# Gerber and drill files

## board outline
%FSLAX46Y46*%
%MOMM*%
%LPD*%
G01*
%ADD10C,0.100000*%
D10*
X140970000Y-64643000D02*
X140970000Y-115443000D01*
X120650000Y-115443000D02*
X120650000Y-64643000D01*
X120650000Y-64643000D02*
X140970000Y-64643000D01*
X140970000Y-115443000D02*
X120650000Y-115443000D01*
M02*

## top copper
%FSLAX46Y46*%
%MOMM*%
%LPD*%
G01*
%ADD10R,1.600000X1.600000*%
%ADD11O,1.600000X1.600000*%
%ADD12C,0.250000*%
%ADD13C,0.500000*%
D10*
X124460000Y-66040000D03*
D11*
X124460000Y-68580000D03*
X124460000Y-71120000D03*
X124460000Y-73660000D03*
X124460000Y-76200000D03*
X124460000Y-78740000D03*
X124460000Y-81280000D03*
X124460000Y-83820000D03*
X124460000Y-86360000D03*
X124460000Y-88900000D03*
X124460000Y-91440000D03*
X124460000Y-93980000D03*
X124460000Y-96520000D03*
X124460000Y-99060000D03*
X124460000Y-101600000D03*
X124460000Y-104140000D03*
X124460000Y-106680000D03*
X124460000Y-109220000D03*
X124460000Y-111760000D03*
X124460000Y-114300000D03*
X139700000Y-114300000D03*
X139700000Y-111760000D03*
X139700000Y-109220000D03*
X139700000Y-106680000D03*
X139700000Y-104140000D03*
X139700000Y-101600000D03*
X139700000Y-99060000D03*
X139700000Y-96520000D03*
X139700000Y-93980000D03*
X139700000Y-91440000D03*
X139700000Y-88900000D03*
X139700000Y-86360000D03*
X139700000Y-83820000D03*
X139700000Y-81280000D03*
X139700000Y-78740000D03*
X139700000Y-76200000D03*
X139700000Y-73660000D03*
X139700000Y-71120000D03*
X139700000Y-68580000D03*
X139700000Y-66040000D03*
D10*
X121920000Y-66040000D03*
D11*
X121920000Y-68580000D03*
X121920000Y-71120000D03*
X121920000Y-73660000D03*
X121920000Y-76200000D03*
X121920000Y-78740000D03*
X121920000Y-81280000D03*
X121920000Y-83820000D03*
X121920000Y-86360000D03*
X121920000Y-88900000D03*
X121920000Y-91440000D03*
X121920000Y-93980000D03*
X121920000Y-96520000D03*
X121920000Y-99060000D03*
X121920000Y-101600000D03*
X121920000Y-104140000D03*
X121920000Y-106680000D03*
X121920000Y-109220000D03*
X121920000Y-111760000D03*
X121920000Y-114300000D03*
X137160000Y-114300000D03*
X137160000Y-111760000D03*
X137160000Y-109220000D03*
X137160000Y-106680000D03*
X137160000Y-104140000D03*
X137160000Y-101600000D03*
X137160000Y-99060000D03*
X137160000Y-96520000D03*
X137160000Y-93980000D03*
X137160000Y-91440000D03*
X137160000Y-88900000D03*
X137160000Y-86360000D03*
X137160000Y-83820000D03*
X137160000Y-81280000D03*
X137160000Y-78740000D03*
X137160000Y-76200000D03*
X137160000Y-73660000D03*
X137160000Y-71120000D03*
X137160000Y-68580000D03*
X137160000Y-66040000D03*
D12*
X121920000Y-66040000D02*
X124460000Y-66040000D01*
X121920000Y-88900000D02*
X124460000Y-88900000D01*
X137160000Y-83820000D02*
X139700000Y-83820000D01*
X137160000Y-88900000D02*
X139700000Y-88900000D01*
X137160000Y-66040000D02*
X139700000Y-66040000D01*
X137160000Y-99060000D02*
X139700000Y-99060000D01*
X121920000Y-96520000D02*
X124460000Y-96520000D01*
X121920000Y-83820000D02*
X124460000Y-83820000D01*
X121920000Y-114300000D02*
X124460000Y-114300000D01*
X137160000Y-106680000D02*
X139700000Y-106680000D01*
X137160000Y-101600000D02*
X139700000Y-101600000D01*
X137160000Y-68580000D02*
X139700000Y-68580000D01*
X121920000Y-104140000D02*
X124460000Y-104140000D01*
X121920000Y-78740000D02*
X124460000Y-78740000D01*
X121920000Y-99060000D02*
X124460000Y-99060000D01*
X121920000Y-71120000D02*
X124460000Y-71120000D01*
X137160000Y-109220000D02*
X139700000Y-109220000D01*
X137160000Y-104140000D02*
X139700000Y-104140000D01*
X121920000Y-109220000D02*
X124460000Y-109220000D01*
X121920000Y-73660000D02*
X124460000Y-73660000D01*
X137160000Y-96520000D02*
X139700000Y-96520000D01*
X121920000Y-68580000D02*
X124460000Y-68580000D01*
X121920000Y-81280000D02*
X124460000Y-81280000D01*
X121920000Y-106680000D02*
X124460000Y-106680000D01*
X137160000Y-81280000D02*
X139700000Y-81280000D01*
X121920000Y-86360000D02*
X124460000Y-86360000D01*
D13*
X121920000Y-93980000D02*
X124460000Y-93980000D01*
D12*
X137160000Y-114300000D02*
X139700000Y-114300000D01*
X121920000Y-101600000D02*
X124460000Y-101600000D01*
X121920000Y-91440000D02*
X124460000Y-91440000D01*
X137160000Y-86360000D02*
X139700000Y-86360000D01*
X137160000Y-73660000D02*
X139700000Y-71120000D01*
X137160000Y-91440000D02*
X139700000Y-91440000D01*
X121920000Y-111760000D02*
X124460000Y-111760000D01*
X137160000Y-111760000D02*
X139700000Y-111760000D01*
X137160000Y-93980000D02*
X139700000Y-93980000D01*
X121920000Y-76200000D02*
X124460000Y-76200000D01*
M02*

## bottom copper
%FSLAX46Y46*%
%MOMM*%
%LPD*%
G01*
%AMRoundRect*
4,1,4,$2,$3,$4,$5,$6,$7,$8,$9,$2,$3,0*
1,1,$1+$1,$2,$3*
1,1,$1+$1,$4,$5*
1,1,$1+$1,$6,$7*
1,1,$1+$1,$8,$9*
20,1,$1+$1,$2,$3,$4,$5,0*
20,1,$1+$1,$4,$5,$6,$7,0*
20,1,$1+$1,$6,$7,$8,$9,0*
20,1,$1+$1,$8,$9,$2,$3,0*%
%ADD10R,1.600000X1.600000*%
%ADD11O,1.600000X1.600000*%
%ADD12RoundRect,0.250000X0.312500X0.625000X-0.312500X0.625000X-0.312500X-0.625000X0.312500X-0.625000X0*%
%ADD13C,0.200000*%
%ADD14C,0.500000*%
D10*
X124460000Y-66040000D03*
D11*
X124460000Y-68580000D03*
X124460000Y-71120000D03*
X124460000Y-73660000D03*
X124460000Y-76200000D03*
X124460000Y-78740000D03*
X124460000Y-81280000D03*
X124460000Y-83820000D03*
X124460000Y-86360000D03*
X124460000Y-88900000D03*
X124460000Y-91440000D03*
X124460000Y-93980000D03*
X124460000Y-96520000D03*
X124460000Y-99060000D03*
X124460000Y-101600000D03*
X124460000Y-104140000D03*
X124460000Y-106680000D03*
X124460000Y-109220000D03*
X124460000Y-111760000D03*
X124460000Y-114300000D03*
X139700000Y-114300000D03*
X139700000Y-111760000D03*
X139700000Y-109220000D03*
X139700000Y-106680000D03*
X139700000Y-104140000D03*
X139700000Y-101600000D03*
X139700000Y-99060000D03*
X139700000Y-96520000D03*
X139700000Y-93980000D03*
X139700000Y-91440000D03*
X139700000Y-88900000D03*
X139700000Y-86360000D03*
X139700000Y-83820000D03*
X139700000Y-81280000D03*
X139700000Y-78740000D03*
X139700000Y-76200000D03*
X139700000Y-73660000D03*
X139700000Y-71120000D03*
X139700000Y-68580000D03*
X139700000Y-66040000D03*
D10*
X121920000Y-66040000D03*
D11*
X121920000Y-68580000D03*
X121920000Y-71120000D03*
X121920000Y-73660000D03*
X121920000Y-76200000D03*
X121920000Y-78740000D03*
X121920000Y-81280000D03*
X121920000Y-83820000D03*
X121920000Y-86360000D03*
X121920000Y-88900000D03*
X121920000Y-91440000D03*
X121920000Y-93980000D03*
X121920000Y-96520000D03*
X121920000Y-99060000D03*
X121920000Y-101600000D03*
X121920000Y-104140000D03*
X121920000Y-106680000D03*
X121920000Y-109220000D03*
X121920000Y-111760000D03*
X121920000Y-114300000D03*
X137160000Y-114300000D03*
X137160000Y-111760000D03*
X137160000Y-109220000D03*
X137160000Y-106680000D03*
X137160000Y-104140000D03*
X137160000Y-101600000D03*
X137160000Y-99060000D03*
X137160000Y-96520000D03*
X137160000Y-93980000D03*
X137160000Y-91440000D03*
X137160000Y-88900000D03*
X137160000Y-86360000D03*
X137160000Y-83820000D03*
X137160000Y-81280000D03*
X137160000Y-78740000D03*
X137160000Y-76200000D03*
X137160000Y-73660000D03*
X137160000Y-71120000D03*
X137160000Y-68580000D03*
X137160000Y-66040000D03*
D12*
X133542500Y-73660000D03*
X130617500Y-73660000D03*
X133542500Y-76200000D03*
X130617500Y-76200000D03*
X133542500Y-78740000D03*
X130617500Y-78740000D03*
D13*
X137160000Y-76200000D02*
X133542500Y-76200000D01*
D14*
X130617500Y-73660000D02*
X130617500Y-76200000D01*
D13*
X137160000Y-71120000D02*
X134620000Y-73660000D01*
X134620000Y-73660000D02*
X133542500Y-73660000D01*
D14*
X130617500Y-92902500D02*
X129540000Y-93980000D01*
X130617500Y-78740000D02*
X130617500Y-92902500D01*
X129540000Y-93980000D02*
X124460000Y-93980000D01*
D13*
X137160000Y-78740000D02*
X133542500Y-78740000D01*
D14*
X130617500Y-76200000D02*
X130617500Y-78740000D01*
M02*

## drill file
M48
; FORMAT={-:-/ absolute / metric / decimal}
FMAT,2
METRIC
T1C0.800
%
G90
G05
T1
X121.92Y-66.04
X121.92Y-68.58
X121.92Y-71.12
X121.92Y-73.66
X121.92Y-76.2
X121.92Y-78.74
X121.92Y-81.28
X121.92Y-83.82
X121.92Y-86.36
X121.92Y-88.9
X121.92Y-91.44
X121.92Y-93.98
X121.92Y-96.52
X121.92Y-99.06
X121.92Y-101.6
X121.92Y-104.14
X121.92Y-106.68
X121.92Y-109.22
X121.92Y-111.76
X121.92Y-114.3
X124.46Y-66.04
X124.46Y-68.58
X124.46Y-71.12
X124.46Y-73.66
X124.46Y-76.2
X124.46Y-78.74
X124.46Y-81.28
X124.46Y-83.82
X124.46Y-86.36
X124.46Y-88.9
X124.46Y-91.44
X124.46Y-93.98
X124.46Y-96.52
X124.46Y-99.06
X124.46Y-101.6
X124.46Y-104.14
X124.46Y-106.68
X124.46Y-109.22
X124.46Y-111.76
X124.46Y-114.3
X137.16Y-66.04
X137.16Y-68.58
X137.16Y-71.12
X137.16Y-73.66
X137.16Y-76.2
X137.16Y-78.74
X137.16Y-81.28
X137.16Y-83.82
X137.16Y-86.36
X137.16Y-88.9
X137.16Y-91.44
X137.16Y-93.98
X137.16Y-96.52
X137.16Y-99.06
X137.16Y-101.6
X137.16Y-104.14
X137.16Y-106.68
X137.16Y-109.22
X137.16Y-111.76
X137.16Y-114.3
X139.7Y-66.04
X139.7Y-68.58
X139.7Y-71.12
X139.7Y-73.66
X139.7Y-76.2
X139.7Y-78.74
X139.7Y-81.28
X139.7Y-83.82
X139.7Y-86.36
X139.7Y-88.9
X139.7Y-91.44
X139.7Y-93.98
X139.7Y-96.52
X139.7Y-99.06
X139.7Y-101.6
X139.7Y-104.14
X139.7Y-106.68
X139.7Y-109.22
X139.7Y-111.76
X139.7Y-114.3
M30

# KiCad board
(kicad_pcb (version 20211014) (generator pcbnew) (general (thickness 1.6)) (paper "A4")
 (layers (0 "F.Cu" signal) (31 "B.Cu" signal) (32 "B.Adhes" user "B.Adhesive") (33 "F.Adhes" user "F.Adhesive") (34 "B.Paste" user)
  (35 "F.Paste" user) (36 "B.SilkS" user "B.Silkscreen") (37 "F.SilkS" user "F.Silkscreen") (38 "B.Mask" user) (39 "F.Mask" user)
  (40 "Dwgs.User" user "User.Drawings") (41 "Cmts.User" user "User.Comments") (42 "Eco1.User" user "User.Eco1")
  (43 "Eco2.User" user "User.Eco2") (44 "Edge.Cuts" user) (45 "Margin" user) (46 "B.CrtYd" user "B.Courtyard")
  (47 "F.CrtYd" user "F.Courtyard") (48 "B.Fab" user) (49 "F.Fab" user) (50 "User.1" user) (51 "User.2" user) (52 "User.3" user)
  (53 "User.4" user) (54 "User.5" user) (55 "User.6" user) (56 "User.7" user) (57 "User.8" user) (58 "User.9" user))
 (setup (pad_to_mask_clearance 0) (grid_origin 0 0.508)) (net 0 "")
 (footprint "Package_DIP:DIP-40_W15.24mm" (layer "F.Cu") (at 124.46 66.04)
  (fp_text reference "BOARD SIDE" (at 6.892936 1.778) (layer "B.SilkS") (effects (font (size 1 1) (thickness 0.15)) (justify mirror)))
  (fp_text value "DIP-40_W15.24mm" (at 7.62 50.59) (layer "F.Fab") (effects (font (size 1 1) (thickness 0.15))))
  (pad "1" thru_hole rect (at 0 0) (size 1.6 1.6) (drill 0.8) (layers *.Cu *.Mask))
  (pad "2" thru_hole oval (at 0 2.54) (size 1.6 1.6) (drill 0.8) (layers *.Cu *.Mask))
  (pad "3" thru_hole oval (at 0 5.08) (size 1.6 1.6) (drill 0.8) (layers *.Cu *.Mask))
  (pad "4" thru_hole oval (at 0 7.62) (size 1.6 1.6) (drill 0.8) (layers *.Cu *.Mask))
  (pad "5" thru_hole oval (at 0 10.16) (size 1.6 1.6) (drill 0.8) (layers *.Cu *.Mask))
  (pad "6" thru_hole oval (at 0 12.7) (size 1.6 1.6) (drill 0.8) (layers *.Cu *.Mask))
  (pad "7" thru_hole oval (at 0 15.24) (size 1.6 1.6) (drill 0.8) (layers *.Cu *.Mask))
  (pad "8" thru_hole oval (at 0 17.78) (size 1.6 1.6) (drill 0.8) (layers *.Cu *.Mask))
  (pad "9" thru_hole oval (at 0 20.32) (size 1.6 1.6) (drill 0.8) (layers *.Cu *.Mask))
  (pad "10" thru_hole oval (at 0 22.86) (size 1.6 1.6) (drill 0.8) (layers *.Cu *.Mask))
  (pad "11" thru_hole oval (at 0 25.4) (size 1.6 1.6) (drill 0.8) (layers *.Cu *.Mask))
  (pad "12" thru_hole oval (at 0 27.94) (size 1.6 1.6) (drill 0.8) (layers *.Cu *.Mask))
  (pad "13" thru_hole oval (at 0 30.48) (size 1.6 1.6) (drill 0.8) (layers *.Cu *.Mask))
  (pad "14" thru_hole oval (at 0 33.02) (size 1.6 1.6) (drill 0.8) (layers *.Cu *.Mask))
  (pad "15" thru_hole oval (at 0 35.56) (size 1.6 1.6) (drill 0.8) (layers *.Cu *.Mask))
  (pad "16" thru_hole oval (at 0 38.1) (size 1.6 1.6) (drill 0.8) (layers *.Cu *.Mask))
  (pad "17" thru_hole oval (at 0 40.64) (size 1.6 1.6) (drill 0.8) (layers *.Cu *.Mask))
  (pad "18" thru_hole oval (at 0 43.18) (size 1.6 1.6) (drill 0.8) (layers *.Cu *.Mask))
  (pad "19" thru_hole oval (at 0 45.72) (size 1.6 1.6) (drill 0.8) (layers *.Cu *.Mask))
  (pad "20" thru_hole oval (at 0 48.26) (size 1.6 1.6) (drill 0.8) (layers *.Cu *.Mask))
  (pad "21" thru_hole oval (at 15.24 48.26) (size 1.6 1.6) (drill 0.8) (layers *.Cu *.Mask))
  (pad "22" thru_hole oval (at 15.24 45.72) (size 1.6 1.6) (drill 0.8) (layers *.Cu *.Mask))
  (pad "23" thru_hole oval (at 15.24 43.18) (size 1.6 1.6) (drill 0.8) (layers *.Cu *.Mask))
  (pad "24" thru_hole oval (at 15.24 40.64) (size 1.6 1.6) (drill 0.8) (layers *.Cu *.Mask))
  (pad "25" thru_hole oval (at 15.24 38.1) (size 1.6 1.6) (drill 0.8) (layers *.Cu *.Mask))
  (pad "26" thru_hole oval (at 15.24 35.56) (size 1.6 1.6) (drill 0.8) (layers *.Cu *.Mask))
  (pad "27" thru_hole oval (at 15.24 33.02) (size 1.6 1.6) (drill 0.8) (layers *.Cu *.Mask))
  (pad "28" thru_hole oval (at 15.24 30.48) (size 1.6 1.6) (drill 0.8) (layers *.Cu *.Mask))
  (pad "29" thru_hole oval (at 15.24 27.94) (size 1.6 1.6) (drill 0.8) (layers *.Cu *.Mask))
  (pad "30" thru_hole oval (at 15.24 25.4) (size 1.6 1.6) (drill 0.8) (layers *.Cu *.Mask))
  (pad "31" thru_hole oval (at 15.24 22.86) (size 1.6 1.6) (drill 0.8) (layers *.Cu *.Mask))
  (pad "32" thru_hole oval (at 15.24 20.32) (size 1.6 1.6) (drill 0.8) (layers *.Cu *.Mask))
  (pad "33" thru_hole oval (at 15.24 17.78) (size 1.6 1.6) (drill 0.8) (layers *.Cu *.Mask))
  (pad "34" thru_hole oval (at 15.24 15.24) (size 1.6 1.6) (drill 0.8) (layers *.Cu *.Mask))
  (pad "35" thru_hole oval (at 15.24 12.7) (size 1.6 1.6) (drill 0.8) (layers *.Cu *.Mask))
  (pad "36" thru_hole oval (at 15.24 10.16) (size 1.6 1.6) (drill 0.8) (layers *.Cu *.Mask))
  (pad "37" thru_hole oval (at 15.24 7.62) (size 1.6 1.6) (drill 0.8) (layers *.Cu *.Mask))
  (pad "38" thru_hole oval (at 15.24 5.08) (size 1.6 1.6) (drill 0.8) (layers *.Cu *.Mask))
  (pad "39" thru_hole oval (at 15.24 2.54) (size 1.6 1.6) (drill 0.8) (layers *.Cu *.Mask))
  (pad "40" thru_hole oval (at 15.24 0) (size 1.6 1.6) (drill 0.8) (layers *.Cu *.Mask)))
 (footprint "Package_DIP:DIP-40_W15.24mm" (layer "F.Cu") (at 121.92 66.04)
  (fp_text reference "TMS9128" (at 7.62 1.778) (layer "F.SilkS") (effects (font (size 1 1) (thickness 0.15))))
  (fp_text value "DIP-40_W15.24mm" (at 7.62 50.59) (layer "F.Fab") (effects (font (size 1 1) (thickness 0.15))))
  (pad "1" thru_hole rect (at 0 0) (size 1.6 1.6) (drill 0.8) (layers *.Cu *.Mask))
  (pad "2" thru_hole oval (at 0 2.54) (size 1.6 1.6) (drill 0.8) (layers *.Cu *.Mask))
  (pad "3" thru_hole oval (at 0 5.08) (size 1.6 1.6) (drill 0.8) (layers *.Cu *.Mask))
  (pad "4" thru_hole oval (at 0 7.62) (size 1.6 1.6) (drill 0.8) (layers *.Cu *.Mask))
  (pad "5" thru_hole oval (at 0 10.16) (size 1.6 1.6) (drill 0.8) (layers *.Cu *.Mask))
  (pad "6" thru_hole oval (at 0 12.7) (size 1.6 1.6) (drill 0.8) (layers *.Cu *.Mask))
  (pad "7" thru_hole oval (at 0 15.24) (size 1.6 1.6) (drill 0.8) (layers *.Cu *.Mask))
  (pad "8" thru_hole oval (at 0 17.78) (size 1.6 1.6) (drill 0.8) (layers *.Cu *.Mask))
  (pad "9" thru_hole oval (at 0 20.32) (size 1.6 1.6) (drill 0.8) (layers *.Cu *.Mask))
  (pad "10" thru_hole oval (at 0 22.86) (size 1.6 1.6) (drill 0.8) (layers *.Cu *.Mask))
  (pad "11" thru_hole oval (at 0 25.4) (size 1.6 1.6) (drill 0.8) (layers *.Cu *.Mask))
  (pad "12" thru_hole oval (at 0 27.94) (size 1.6 1.6) (drill 0.8) (layers *.Cu *.Mask))
  (pad "13" thru_hole oval (at 0 30.48) (size 1.6 1.6) (drill 0.8) (layers *.Cu *.Mask))
  (pad "14" thru_hole oval (at 0 33.02) (size 1.6 1.6) (drill 0.8) (layers *.Cu *.Mask))
  (pad "15" thru_hole oval (at 0 35.56) (size 1.6 1.6) (drill 0.8) (layers *.Cu *.Mask))
  (pad "16" thru_hole oval (at 0 38.1) (size 1.6 1.6) (drill 0.8) (layers *.Cu *.Mask))
  (pad "17" thru_hole oval (at 0 40.64) (size 1.6 1.6) (drill 0.8) (layers *.Cu *.Mask))
  (pad "18" thru_hole oval (at 0 43.18) (size 1.6 1.6) (drill 0.8) (layers *.Cu *.Mask))
  (pad "19" thru_hole oval (at 0 45.72) (size 1.6 1.6) (drill 0.8) (layers *.Cu *.Mask))
  (pad "20" thru_hole oval (at 0 48.26) (size 1.6 1.6) (drill 0.8) (layers *.Cu *.Mask))
  (pad "21" thru_hole oval (at 15.24 48.26) (size 1.6 1.6) (drill 0.8) (layers *.Cu *.Mask))
  (pad "22" thru_hole oval (at 15.24 45.72) (size 1.6 1.6) (drill 0.8) (layers *.Cu *.Mask))
  (pad "23" thru_hole oval (at 15.24 43.18) (size 1.6 1.6) (drill 0.8) (layers *.Cu *.Mask))
  (pad "24" thru_hole oval (at 15.24 40.64) (size 1.6 1.6) (drill 0.8) (layers *.Cu *.Mask))
  (pad "25" thru_hole oval (at 15.24 38.1) (size 1.6 1.6) (drill 0.8) (layers *.Cu *.Mask))
  (pad "26" thru_hole oval (at 15.24 35.56) (size 1.6 1.6) (drill 0.8) (layers *.Cu *.Mask))
  (pad "27" thru_hole oval (at 15.24 33.02) (size 1.6 1.6) (drill 0.8) (layers *.Cu *.Mask))
  (pad "28" thru_hole oval (at 15.24 30.48) (size 1.6 1.6) (drill 0.8) (layers *.Cu *.Mask))
  (pad "29" thru_hole oval (at 15.24 27.94) (size 1.6 1.6) (drill 0.8) (layers *.Cu *.Mask))
  (pad "30" thru_hole oval (at 15.24 25.4) (size 1.6 1.6) (drill 0.8) (layers *.Cu *.Mask))
  (pad "31" thru_hole oval (at 15.24 22.86) (size 1.6 1.6) (drill 0.8) (layers *.Cu *.Mask))
  (pad "32" thru_hole oval (at 15.24 20.32) (size 1.6 1.6) (drill 0.8) (layers *.Cu *.Mask))
  (pad "33" thru_hole oval (at 15.24 17.78) (size 1.6 1.6) (drill 0.8) (layers *.Cu *.Mask))
  (pad "34" thru_hole oval (at 15.24 15.24) (size 1.6 1.6) (drill 0.8) (layers *.Cu *.Mask))
  (pad "35" thru_hole oval (at 15.24 12.7) (size 1.6 1.6) (drill 0.8) (layers *.Cu *.Mask))
  (pad "36" thru_hole oval (at 15.24 10.16) (size 1.6 1.6) (drill 0.8) (layers *.Cu *.Mask))
  (pad "37" thru_hole oval (at 15.24 7.62) (size 1.6 1.6) (drill 0.8) (layers *.Cu *.Mask))
  (pad "38" thru_hole oval (at 15.24 5.08) (size 1.6 1.6) (drill 0.8) (layers *.Cu *.Mask))
  (pad "39" thru_hole oval (at 15.24 2.54) (size 1.6 1.6) (drill 0.8) (layers *.Cu *.Mask))
  (pad "40" thru_hole oval (at 15.24 0) (size 1.6 1.6) (drill 0.8) (layers *.Cu *.Mask)))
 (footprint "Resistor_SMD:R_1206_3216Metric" (layer "B.Cu") (at 132.08 73.66 180)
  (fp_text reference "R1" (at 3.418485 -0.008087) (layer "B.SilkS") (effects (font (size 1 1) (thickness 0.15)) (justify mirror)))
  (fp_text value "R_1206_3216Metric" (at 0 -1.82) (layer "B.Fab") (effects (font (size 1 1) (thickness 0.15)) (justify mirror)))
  (pad "1" smd roundrect (at -1.4625 0 180) (size 1.125 1.75) (layers "B.Cu" "B.Paste" "B.Mask") (roundrect_rratio 0.2222222222))
  (pad "2" smd roundrect (at 1.4625 0 180) (size 1.125 1.75) (layers "B.Cu" "B.Paste" "B.Mask") (roundrect_rratio 0.2222222222)))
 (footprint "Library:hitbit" (layer "B.Cu") (at 130.81 103.378 90)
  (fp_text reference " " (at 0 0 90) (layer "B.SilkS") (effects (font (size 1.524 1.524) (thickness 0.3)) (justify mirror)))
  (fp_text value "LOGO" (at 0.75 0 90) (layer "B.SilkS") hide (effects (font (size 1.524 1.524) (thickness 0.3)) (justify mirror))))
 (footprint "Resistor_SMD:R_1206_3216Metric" (layer "B.Cu") (at 132.08 76.2 180)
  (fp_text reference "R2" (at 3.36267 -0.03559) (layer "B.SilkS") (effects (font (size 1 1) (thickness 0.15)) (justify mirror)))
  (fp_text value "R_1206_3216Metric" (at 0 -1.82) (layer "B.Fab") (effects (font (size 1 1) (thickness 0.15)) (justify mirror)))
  (pad "1" smd roundrect (at -1.4625 0 180) (size 1.125 1.75) (layers "B.Cu" "B.Paste" "B.Mask") (roundrect_rratio 0.2222222222))
  (pad "2" smd roundrect (at 1.4625 0 180) (size 1.125 1.75) (layers "B.Cu" "B.Paste" "B.Mask") (roundrect_rratio 0.2222222222)))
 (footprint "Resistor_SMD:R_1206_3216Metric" (layer "B.Cu") (at 132.08 78.74 180)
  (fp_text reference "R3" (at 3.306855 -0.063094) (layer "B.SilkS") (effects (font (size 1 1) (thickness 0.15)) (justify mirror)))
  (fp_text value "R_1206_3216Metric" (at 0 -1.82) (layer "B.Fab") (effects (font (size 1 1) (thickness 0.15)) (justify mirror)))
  (pad "1" smd roundrect (at -1.4625 0 180) (size 1.125 1.75) (layers "B.Cu" "B.Paste" "B.Mask") (roundrect_rratio 0.2222222222))
  (pad "2" smd roundrect (at 1.4625 0 180) (size 1.125 1.75) (layers "B.Cu" "B.Paste" "B.Mask") (roundrect_rratio 0.2222222222)))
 (gr_line (start 140.97 64.643) (end 140.97 115.443) (layer "Edge.Cuts") (width 0.1))
 (gr_line (start 120.65 115.443) (end 120.65 64.643) (layer "Edge.Cuts") (width 0.1))
 (gr_line (start 120.65 64.643) (end 140.97 64.643) (layer "Edge.Cuts") (width 0.1))
 (gr_line (start 140.97 115.443) (end 120.65 115.443) (layer "Edge.Cuts") (width 0.1))
 (segment (start 121.92 66.04) (end 124.46 66.04) (width 0.25) (layer "F.Cu") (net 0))
 (segment (start 121.92 88.9) (end 124.46 88.9) (width 0.25) (layer "F.Cu") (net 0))
 (segment (start 137.16 83.82) (end 139.7 83.82) (width 0.25) (layer "F.Cu") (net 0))
 (segment (start 137.16 88.9) (end 139.7 88.9) (width 0.25) (layer "F.Cu") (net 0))
 (segment (start 137.16 66.04) (end 139.7 66.04) (width 0.25) (layer "F.Cu") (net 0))
 (segment (start 137.16 99.06) (end 139.7 99.06) (width 0.25) (layer "F.Cu") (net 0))
 (segment (start 121.92 96.52) (end 124.46 96.52) (width 0.25) (layer "F.Cu") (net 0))
 (segment (start 121.92 83.82) (end 124.46 83.82) (width 0.25) (layer "F.Cu") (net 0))
 (segment (start 121.92 114.3) (end 124.46 114.3) (width 0.25) (layer "F.Cu") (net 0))
 (segment (start 137.16 106.68) (end 139.7 106.68) (width 0.25) (layer "F.Cu") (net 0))
 (segment (start 137.16 101.6) (end 139.7 101.6) (width 0.25) (layer "F.Cu") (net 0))
 (segment (start 137.16 68.58) (end 139.7 68.58) (width 0.25) (layer "F.Cu") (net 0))
 (segment (start 121.92 104.14) (end 124.46 104.14) (width 0.25) (layer "F.Cu") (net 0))
 (segment (start 121.92 78.74) (end 124.46 78.74) (width 0.25) (layer "F.Cu") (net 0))
 (segment (start 121.92 99.06) (end 124.46 99.06) (width 0.25) (layer "F.Cu") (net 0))
 (segment (start 121.92 71.12) (end 124.46 71.12) (width 0.25) (layer "F.Cu") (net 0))
 (segment (start 137.16 109.22) (end 139.7 109.22) (width 0.25) (layer "F.Cu") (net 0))
 (segment (start 137.16 104.14) (end 139.7 104.14) (width 0.25) (layer "F.Cu") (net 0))
 (segment (start 121.92 109.22) (end 124.46 109.22) (width 0.25) (layer "F.Cu") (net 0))
 (segment (start 121.92 73.66) (end 124.46 73.66) (width 0.25) (layer "F.Cu") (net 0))
 (segment (start 137.16 96.52) (end 139.7 96.52) (width 0.25) (layer "F.Cu") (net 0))
 (segment (start 121.92 68.58) (end 124.46 68.58) (width 0.25) (layer "F.Cu") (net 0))
 (segment (start 121.92 81.28) (end 124.46 81.28) (width 0.25) (layer "F.Cu") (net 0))
 (segment (start 121.92 106.68) (end 124.46 106.68) (width 0.25) (layer "F.Cu") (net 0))
 (segment (start 137.16 81.28) (end 139.7 81.28) (width 0.25) (layer "F.Cu") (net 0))
 (segment (start 121.92 86.36) (end 124.46 86.36) (width 0.25) (layer "F.Cu") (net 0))
 (segment (start 121.92 93.98) (end 124.46 93.98) (width 0.5) (layer "F.Cu") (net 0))
 (segment (start 137.16 114.3) (end 139.7 114.3) (width 0.25) (layer "F.Cu") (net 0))
 (segment (start 121.92 101.6) (end 124.46 101.6) (width 0.25) (layer "F.Cu") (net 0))
 (segment (start 121.92 91.44) (end 124.46 91.44) (width 0.25) (layer "F.Cu") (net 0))
 (segment (start 137.16 86.36) (end 139.7 86.36) (width 0.25) (layer "F.Cu") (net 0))
 (segment (start 137.16 73.66) (end 139.7 71.12) (width 0.25) (layer "F.Cu") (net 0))
 (segment (start 137.16 91.44) (end 139.7 91.44) (width 0.25) (layer "F.Cu") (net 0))
 (segment (start 121.92 111.76) (end 124.46 111.76) (width 0.25) (layer "F.Cu") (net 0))
 (segment (start 137.16 111.76) (end 139.7 111.76) (width 0.25) (layer "F.Cu") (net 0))
 (segment (start 137.16 93.98) (end 139.7 93.98) (width 0.25) (layer "F.Cu") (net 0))
 (segment (start 121.92 76.2) (end 124.46 76.2) (width 0.25) (layer "F.Cu") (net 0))
 (segment (start 137.16 76.2) (end 133.5425 76.2) (width 0.2) (layer "B.Cu") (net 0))
 (segment (start 130.6175 73.66) (end 130.6175 76.2) (width 0.5) (layer "B.Cu") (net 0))
 (segment (start 137.16 71.12) (end 134.62 73.66) (width 0.2) (layer "B.Cu") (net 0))
 (segment (start 134.62 73.66) (end 133.5425 73.66) (width 0.2) (layer "B.Cu") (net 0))
 (segment (start 130.6175 92.9025) (end 129.54 93.98) (width 0.5) (layer "B.Cu") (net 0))
 (segment (start 130.6175 78.74) (end 130.6175 92.9025) (width 0.5) (layer "B.Cu") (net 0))
 (segment (start 129.54 93.98) (end 124.46 93.98) (width 0.5) (layer "B.Cu") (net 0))
 (segment (start 137.16 78.74) (end 133.5425 78.74) (width 0.2) (layer "B.Cu") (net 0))
 (segment (start 130.6175 76.2) (end 130.6175 78.74) (width 0.5) (layer "B.Cu") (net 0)))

